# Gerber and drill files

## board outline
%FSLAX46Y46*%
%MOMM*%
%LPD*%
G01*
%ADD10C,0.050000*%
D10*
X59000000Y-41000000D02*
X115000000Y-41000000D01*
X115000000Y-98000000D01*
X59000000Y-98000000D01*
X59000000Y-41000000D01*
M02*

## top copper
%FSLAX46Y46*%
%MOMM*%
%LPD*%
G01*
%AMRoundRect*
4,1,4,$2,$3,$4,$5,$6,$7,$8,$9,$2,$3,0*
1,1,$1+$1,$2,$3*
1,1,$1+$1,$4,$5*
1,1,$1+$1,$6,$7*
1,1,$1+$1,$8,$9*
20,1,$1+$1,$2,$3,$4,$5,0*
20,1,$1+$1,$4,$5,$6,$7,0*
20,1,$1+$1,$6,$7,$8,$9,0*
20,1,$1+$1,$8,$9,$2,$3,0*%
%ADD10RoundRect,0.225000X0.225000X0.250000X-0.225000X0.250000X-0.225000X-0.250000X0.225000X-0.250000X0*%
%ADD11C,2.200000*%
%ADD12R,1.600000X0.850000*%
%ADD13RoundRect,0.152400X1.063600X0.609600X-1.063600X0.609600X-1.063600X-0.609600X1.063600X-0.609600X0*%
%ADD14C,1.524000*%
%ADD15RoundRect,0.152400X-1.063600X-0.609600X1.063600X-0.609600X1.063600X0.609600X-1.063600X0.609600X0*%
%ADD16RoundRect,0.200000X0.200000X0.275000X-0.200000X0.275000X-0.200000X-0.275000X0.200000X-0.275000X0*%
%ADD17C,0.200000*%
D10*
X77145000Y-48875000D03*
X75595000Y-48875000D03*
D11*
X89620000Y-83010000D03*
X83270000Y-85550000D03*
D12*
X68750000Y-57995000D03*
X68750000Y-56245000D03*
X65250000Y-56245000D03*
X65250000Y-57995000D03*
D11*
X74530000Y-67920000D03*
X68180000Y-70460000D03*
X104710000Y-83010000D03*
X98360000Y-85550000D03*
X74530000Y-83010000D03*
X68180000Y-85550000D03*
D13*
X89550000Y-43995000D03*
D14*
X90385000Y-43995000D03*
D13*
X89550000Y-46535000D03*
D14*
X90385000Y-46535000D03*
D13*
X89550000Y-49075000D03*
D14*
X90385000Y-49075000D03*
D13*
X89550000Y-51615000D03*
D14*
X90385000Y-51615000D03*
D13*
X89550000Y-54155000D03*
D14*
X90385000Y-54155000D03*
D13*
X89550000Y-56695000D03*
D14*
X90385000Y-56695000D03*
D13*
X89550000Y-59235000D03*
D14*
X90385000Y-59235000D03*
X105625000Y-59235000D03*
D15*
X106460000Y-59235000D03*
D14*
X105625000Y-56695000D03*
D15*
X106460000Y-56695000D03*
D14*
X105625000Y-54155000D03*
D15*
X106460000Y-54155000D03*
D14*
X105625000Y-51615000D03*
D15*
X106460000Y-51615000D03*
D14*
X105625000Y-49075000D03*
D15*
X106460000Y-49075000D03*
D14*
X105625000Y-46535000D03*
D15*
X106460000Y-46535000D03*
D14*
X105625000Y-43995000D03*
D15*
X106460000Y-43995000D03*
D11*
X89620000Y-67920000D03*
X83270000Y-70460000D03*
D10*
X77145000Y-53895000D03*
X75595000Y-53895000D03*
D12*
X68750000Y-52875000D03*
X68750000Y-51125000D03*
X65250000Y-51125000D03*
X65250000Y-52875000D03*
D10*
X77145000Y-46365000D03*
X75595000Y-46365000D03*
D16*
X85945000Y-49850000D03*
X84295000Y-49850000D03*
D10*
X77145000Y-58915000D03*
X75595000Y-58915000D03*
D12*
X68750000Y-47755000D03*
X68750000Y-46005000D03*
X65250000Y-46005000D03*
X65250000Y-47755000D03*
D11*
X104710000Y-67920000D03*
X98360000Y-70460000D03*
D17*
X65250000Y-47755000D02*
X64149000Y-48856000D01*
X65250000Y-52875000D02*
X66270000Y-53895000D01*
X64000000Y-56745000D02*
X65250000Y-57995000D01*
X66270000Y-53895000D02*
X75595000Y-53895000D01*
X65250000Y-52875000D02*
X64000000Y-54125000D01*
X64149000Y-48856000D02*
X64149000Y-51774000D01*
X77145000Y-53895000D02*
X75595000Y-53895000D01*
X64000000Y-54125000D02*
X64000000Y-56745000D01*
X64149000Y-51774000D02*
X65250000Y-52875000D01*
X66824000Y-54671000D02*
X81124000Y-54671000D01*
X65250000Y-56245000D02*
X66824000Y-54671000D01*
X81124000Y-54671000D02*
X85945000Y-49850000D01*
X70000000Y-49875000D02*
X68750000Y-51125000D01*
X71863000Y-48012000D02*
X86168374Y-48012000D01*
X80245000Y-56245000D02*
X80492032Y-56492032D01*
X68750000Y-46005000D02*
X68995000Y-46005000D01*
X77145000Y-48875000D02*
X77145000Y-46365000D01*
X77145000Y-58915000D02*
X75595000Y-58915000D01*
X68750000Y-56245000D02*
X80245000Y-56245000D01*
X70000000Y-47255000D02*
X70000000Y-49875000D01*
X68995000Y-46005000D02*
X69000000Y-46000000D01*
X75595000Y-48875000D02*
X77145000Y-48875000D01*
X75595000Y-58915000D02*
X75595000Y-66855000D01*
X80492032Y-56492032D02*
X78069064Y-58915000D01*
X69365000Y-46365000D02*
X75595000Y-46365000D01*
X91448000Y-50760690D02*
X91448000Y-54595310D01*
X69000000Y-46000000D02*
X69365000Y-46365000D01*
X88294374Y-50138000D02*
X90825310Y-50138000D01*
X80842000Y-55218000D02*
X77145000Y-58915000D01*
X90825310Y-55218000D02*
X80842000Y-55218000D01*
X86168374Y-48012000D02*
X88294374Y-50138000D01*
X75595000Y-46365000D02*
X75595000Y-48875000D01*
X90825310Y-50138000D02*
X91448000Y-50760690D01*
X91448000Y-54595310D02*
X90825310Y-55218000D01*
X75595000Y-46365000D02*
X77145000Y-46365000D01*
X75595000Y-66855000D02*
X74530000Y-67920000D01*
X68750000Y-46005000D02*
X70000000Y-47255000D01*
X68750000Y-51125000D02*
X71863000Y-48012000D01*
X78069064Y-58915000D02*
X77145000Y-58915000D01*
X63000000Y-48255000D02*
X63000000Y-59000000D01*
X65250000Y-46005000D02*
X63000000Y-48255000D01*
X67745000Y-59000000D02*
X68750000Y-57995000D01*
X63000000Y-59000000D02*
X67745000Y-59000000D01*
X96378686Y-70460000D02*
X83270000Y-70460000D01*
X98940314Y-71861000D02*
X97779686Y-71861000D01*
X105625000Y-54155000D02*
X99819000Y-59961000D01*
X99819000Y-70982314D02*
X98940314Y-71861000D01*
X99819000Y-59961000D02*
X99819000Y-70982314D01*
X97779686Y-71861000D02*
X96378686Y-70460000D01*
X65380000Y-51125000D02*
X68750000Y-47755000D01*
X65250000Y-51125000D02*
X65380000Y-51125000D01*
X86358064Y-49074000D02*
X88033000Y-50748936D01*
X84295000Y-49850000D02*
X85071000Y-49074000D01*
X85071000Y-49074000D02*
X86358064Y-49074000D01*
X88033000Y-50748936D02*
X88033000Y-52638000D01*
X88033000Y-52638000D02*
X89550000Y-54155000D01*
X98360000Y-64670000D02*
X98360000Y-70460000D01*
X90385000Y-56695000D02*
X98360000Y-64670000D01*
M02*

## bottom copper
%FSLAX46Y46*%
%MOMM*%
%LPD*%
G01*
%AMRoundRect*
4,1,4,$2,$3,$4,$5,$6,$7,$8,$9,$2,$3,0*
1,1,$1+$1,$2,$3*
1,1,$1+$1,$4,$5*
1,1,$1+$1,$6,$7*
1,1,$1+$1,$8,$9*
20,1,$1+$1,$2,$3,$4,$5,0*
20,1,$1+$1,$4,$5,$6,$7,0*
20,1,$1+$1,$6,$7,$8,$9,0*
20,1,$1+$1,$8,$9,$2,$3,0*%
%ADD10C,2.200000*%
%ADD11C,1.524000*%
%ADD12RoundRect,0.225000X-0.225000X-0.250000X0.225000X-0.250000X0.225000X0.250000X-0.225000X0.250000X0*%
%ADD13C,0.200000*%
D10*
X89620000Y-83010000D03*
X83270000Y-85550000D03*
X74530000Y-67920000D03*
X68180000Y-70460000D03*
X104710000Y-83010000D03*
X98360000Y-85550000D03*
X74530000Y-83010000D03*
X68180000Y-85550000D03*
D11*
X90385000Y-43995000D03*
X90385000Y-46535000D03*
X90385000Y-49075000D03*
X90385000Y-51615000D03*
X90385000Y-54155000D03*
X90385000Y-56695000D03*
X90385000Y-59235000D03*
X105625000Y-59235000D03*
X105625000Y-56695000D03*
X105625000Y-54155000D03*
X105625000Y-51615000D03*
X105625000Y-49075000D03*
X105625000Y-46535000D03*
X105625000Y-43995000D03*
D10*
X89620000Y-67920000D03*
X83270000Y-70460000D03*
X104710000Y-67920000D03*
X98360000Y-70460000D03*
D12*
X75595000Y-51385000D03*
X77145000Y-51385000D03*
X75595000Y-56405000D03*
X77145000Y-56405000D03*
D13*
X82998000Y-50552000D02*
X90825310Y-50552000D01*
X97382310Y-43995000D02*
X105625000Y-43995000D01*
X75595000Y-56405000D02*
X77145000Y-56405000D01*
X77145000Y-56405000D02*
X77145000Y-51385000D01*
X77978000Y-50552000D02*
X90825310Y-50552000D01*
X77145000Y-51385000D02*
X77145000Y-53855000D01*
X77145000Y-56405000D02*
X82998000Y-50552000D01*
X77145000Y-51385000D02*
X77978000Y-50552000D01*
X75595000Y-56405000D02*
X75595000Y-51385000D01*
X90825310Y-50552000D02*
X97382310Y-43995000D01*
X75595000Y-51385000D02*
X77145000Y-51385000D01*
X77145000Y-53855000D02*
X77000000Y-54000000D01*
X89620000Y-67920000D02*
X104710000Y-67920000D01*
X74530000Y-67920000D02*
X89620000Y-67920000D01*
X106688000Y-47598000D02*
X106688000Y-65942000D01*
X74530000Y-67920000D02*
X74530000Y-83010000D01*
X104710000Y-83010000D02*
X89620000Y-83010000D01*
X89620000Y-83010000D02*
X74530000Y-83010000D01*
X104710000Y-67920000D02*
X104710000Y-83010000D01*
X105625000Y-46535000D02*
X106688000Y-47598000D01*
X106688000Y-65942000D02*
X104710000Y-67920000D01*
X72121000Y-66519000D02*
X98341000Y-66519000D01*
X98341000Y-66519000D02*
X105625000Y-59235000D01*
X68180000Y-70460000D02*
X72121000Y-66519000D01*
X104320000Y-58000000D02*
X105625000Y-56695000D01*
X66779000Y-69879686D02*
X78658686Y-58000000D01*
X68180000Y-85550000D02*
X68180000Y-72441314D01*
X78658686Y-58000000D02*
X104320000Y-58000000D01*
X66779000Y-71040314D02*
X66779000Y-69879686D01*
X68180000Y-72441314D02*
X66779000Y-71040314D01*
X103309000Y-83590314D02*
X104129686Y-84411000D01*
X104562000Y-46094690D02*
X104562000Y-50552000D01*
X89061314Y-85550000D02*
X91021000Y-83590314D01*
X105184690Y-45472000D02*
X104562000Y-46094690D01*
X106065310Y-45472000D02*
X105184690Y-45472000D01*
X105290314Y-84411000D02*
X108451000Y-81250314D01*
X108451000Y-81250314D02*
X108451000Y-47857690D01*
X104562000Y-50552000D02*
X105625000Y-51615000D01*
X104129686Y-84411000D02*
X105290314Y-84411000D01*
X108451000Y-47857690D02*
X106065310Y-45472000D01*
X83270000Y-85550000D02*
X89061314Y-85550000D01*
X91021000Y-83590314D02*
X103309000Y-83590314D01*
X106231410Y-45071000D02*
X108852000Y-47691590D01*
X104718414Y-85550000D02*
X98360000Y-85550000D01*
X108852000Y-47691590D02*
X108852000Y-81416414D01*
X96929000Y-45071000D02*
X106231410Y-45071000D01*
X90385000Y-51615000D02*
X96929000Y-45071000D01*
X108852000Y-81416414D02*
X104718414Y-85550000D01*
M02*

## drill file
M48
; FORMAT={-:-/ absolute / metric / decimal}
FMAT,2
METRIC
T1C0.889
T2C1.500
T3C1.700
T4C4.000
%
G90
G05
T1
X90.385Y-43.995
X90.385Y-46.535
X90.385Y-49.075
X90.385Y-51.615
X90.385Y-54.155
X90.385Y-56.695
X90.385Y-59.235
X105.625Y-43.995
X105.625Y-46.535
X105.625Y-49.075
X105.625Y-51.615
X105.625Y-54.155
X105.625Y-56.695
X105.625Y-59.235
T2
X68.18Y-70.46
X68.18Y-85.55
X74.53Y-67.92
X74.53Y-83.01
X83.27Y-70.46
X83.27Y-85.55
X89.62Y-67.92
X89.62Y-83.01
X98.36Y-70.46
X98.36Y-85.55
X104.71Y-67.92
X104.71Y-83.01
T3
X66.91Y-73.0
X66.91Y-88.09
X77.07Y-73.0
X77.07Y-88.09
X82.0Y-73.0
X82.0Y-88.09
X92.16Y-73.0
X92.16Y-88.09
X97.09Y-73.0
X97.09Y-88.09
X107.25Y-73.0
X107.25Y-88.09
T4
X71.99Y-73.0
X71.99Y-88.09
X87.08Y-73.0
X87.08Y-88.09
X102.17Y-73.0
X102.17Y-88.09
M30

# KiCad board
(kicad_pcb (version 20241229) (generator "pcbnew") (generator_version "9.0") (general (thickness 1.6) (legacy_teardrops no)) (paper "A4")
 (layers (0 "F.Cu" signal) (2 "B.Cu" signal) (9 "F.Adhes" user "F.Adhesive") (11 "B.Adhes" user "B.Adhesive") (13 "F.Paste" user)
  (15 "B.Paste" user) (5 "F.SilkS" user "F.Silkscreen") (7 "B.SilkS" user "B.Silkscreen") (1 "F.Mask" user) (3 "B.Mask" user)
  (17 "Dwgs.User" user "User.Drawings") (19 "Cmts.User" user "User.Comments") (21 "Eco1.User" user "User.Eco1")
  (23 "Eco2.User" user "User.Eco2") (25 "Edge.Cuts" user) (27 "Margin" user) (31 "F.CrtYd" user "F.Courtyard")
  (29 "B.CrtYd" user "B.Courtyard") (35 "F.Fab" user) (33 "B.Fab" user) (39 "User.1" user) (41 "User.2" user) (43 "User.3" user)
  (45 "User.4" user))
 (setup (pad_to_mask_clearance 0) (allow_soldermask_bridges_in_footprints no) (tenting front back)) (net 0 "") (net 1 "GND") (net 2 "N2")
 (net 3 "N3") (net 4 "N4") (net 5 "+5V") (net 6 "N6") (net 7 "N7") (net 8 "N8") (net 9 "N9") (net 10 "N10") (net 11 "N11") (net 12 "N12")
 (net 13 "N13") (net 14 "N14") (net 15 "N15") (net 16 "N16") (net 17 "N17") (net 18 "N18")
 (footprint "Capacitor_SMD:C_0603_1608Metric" (layer "F.Cu") (at 76.37 48.875 180)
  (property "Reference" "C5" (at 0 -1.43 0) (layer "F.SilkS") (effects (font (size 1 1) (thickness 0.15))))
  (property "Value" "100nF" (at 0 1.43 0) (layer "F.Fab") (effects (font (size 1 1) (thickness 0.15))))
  (pad "1" smd roundrect (at -0.775 0 180) (size 0.9 0.95) (layers "F.Cu" "F.Mask" "F.Paste") (roundrect_rratio 0.25) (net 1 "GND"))
  (pad "2" smd roundrect (at 0.775 0 180) (size 0.9 0.95) (layers "F.Cu" "F.Mask" "F.Paste") (roundrect_rratio 0.25) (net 1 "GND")))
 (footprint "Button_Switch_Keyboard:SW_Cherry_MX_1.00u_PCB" (layer "F.Cu") (at 89.62 83.01)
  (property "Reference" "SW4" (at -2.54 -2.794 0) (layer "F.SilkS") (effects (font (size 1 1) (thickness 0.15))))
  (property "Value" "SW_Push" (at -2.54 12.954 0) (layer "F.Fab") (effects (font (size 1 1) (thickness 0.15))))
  (pad "" np_thru_hole circle (at -7.62 5.08) (size 1.7 1.7) (drill 1.7) (layers "*.Cu" "*.Mask"))
  (pad "" np_thru_hole circle (at -2.54 5.08) (size 4 4) (drill 4) (layers "*.Cu" "*.Mask"))
  (pad "" np_thru_hole circle (at 2.54 5.08) (size 1.7 1.7) (drill 1.7) (layers "*.Cu" "*.Mask"))
  (pad "1" thru_hole circle (at 0 0) (size 2.2 2.2) (drill 1.5) (layers "*.Cu" "*.Mask") (remove_unused_layers no) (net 1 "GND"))
  (pad "2" thru_hole circle (at -6.35 2.54) (size 2.2 2.2) (drill 1.5) (layers "*.Cu" "*.Mask") (remove_unused_layers no) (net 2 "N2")))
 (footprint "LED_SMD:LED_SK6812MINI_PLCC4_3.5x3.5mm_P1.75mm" (layer "F.Cu") (at 67 57.12 180)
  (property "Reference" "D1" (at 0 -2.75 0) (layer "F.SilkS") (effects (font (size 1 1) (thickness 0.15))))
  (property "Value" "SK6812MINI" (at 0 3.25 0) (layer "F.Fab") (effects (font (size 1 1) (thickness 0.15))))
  (pad "1" smd rect (at -1.75 -0.875 180) (size 1.6 0.85) (layers "F.Cu" "F.Mask" "F.Paste") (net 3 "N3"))
  (pad "2" smd rect (at -1.75 0.875 180) (size 1.6 0.85) (layers "F.Cu" "F.Mask" "F.Paste") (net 1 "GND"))
  (pad "3" smd rect (at 1.75 0.875 180) (size 1.6 0.85) (layers "F.Cu" "F.Mask" "F.Paste") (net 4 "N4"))
  (pad "4" smd rect (at 1.75 -0.875 180) (size 1.6 0.85) (layers "F.Cu" "F.Mask" "F.Paste") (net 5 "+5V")))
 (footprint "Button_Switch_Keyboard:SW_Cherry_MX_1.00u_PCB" (layer "F.Cu") (at 74.53 67.92)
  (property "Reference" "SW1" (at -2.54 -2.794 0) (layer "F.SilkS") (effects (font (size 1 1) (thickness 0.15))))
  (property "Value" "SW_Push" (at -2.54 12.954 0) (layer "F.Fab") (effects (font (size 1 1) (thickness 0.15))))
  (pad "" np_thru_hole circle (at -7.62 5.08) (size 1.7 1.7) (drill 1.7) (layers "*.Cu" "*.Mask"))
  (pad "" np_thru_hole circle (at -2.54 5.08) (size 4 4) (drill 4) (layers "*.Cu" "*.Mask"))
  (pad "" np_thru_hole circle (at 2.54 5.08) (size 1.7 1.7) (drill 1.7) (layers "*.Cu" "*.Mask"))
  (pad "1" thru_hole circle (at 0 0) (size 2.2 2.2) (drill 1.5) (layers "*.Cu" "*.Mask") (remove_unused_layers no) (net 1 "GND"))
  (pad "2" thru_hole circle (at -6.35 2.54) (size 2.2 2.2) (drill 1.5) (layers "*.Cu" "*.Mask") (remove_unused_layers no) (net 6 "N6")))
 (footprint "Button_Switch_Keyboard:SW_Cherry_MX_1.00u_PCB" (layer "F.Cu") (at 104.71 83.01)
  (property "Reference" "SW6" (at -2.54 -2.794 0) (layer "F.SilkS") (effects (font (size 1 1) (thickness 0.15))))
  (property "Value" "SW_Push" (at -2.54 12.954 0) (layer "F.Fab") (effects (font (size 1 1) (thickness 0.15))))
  (pad "" np_thru_hole circle (at -7.62 5.08) (size 1.7 1.7) (drill 1.7) (layers "*.Cu" "*.Mask"))
  (pad "" np_thru_hole circle (at -2.54 5.08) (size 4 4) (drill 4) (layers "*.Cu" "*.Mask"))
  (pad "" np_thru_hole circle (at 2.54 5.08) (size 1.7 1.7) (drill 1.7) (layers "*.Cu" "*.Mask"))
  (pad "1" thru_hole circle (at 0 0) (size 2.2 2.2) (drill 1.5) (layers "*.Cu" "*.Mask") (remove_unused_layers no) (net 1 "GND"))
  (pad "2" thru_hole circle (at -6.35 2.54) (size 2.2 2.2) (drill 1.5) (layers "*.Cu" "*.Mask") (remove_unused_layers no) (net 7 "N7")))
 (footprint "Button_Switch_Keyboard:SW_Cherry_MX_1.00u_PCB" (layer "F.Cu") (at 74.53 83.01)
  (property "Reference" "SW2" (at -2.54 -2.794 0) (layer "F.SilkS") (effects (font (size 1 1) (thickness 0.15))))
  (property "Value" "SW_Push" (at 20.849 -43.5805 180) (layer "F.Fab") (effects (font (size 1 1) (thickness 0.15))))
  (pad "" np_thru_hole circle (at -7.62 5.08) (size 1.7 1.7) (drill 1.7) (layers "*.Cu" "*.Mask"))
  (pad "" np_thru_hole circle (at -2.54 5.08) (size 4 4) (drill 4) (layers "*.Cu" "*.Mask"))
  (pad "" np_thru_hole circle (at 2.54 5.08) (size 1.7 1.7) (drill 1.7) (layers "*.Cu" "*.Mask"))
  (pad "1" thru_hole circle (at 0 0) (size 2.2 2.2) (drill 1.5) (layers "*.Cu" "*.Mask") (remove_unused_layers no) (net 1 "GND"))
  (pad "2" thru_hole circle (at -6.35 2.54) (size 2.2 2.2) (drill 1.5) (layers "*.Cu" "*.Mask") (remove_unused_layers no) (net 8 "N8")))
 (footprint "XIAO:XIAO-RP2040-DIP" (layer "F.Cu") (at 98.005 51.615)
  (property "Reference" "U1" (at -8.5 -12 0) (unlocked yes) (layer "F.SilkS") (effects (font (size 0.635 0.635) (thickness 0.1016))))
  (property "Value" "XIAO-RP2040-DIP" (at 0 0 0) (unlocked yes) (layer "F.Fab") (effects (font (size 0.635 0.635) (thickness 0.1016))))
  (pad "1" smd roundrect (at -8.455 -7.62 180) (size 2.432 1.524) (layers "F.Cu" "F.Mask") (roundrect_rratio 0.1) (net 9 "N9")
   (thermal_bridge_angle 45))
  (pad "1" thru_hole circle (at -7.62 -7.62 180) (size 1.524 1.524) (drill 0.889) (layers "*.Cu" "*.Mask") (remove_unused_layers no)
   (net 9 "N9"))
  (pad "2" smd roundrect (at -8.455 -5.08 180) (size 2.432 1.524) (layers "F.Cu" "F.Mask") (roundrect_rratio 0.1) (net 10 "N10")
   (thermal_bridge_angle 45))
  (pad "2" thru_hole circle (at -7.62 -5.08 180) (size 1.524 1.524) (drill 0.889) (layers "*.Cu" "*.Mask") (remove_unused_layers no)
   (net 10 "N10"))
  (pad "3" smd roundrect (at -8.455 -2.54 180) (size 2.432 1.524) (layers "F.Cu" "F.Mask") (roundrect_rratio 0.1) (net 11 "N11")
   (thermal_bridge_angle 45))
  (pad "3" thru_hole circle (at -7.62 -2.54 180) (size 1.524 1.524) (drill 0.889) (layers "*.Cu" "*.Mask") (remove_unused_layers no)
   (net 11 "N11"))
  (pad "4" smd roundrect (at -8.455 0 180) (size 2.432 1.524) (layers "F.Cu" "F.Mask") (roundrect_rratio 0.1) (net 7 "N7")
   (thermal_bridge_angle 45))
  (pad "4" thru_hole circle (at -7.62 0 180) (size 1.524 1.524) (drill 0.889) (layers "*.Cu" "*.Mask") (remove_unused_layers no)
   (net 7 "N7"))
  (pad "5" smd roundrect (at -8.455 2.54 180) (size 2.432 1.524) (layers "F.Cu" "F.Mask") (roundrect_rratio 0.1) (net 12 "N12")
   (thermal_bridge_angle 45))
  (pad "5" thru_hole circle (at -7.62 2.54 180) (size 1.524 1.524) (drill 0.889) (layers "*.Cu" "*.Mask") (remove_unused_layers no)
   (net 12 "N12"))
  (pad "6" smd roundrect (at -8.455 5.08 180) (size 2.432 1.524) (layers "F.Cu" "F.Mask") (roundrect_rratio 0.1) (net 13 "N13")
   (thermal_bridge_angle 45))
  (pad "6" thru_hole circle (at -7.62 5.08 180) (size 1.524 1.524) (drill 0.889) (layers "*.Cu" "*.Mask") (remove_unused_layers no)
   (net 13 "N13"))
  (pad "7" smd roundrect (at -8.455 7.62 180) (size 2.432 1.524) (layers "F.Cu" "F.Mask") (roundrect_rratio 0.1) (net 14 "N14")
   (thermal_bridge_angle 45))
  (pad "7" thru_hole circle (at -7.62 7.62 180) (size 1.524 1.524) (drill 0.889) (layers "*.Cu" "*.Mask") (remove_unused_layers no)
   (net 14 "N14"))
  (pad "8" thru_hole circle (at 7.62 7.62) (size 1.524 1.524) (drill 0.889) (layers "*.Cu" "*.Mask") (remove_unused_layers no) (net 6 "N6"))
  (pad "8" smd roundrect (at 8.455 7.62) (size 2.432 1.524) (layers "F.Cu" "F.Mask") (roundrect_rratio 0.1) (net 6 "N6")
   (thermal_bridge_angle 45))
  (pad "9" thru_hole circle (at 7.62 5.08) (size 1.524 1.524) (drill 0.889) (layers "*.Cu" "*.Mask") (remove_unused_layers no) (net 8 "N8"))
  (pad "9" smd roundrect (at 8.455 5.08) (size 2.432 1.524) (layers "F.Cu" "F.Mask") (roundrect_rratio 0.1) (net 8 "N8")
   (thermal_bridge_angle 45))
  (pad "10" thru_hole circle (at 7.62 2.54) (size 1.524 1.524) (drill 0.889) (layers "*.Cu" "*.Mask") (remove_unused_layers no)
   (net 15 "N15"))
  (pad "10" smd roundrect (at 8.455 2.54) (size 2.432 1.524) (layers "F.Cu" "F.Mask") (roundrect_rratio 0.1) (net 15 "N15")
   (thermal_bridge_angle 45))
  (pad "11" thru_hole circle (at 7.62 0) (size 1.524 1.524) (drill 0.889) (layers "*.Cu" "*.Mask") (remove_unused_layers no) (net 2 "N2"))
  (pad "11" smd roundrect (at 8.455 0) (size 2.432 1.524) (layers "F.Cu" "F.Mask") (roundrect_rratio 0.1) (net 2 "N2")
   (thermal_bridge_angle 45))
  (pad "12" thru_hole circle (at 7.62 -2.54) (size 1.524 1.524) (drill 0.889) (layers "*.Cu" "*.Mask") (remove_unused_layers no)
   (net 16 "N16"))
  (pad "12" smd roundrect (at 8.455 -2.54) (size 2.432 1.524) (layers "F.Cu" "F.Mask") (roundrect_rratio 0.1) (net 16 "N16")
   (thermal_bridge_angle 45))
  (pad "13" thru_hole circle (at 7.62 -5.08) (size 1.524 1.524) (drill 0.889) (layers "*.Cu" "*.Mask") (remove_unused_layers no)
   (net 1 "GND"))
  (pad "13" smd roundrect (at 8.455 -5.08) (size 2.432 1.524) (layers "F.Cu" "F.Mask") (roundrect_rratio 0.1) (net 1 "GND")
   (thermal_bridge_angle 45))
  (pad "14" thru_hole circle (at 7.62 -7.62) (size 1.524 1.524) (drill 0.889) (layers "*.Cu" "*.Mask") (remove_unused_layers no)
   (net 5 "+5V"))
  (pad "14" smd roundrect (at 8.455 -7.62) (size 2.432 1.524) (layers "F.Cu" "F.Mask") (roundrect_rratio 0.1) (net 5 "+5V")
   (thermal_bridge_angle 45)))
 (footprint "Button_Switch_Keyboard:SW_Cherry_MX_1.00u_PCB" (layer "F.Cu") (at 89.62 67.92)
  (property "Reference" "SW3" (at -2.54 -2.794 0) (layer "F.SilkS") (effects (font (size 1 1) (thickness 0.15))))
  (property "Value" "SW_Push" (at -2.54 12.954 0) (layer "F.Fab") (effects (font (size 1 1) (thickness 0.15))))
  (pad "" np_thru_hole circle (at -7.62 5.08) (size 1.7 1.7) (drill 1.7) (layers "*.Cu" "*.Mask"))
  (pad "" np_thru_hole circle (at -2.54 5.08) (size 4 4) (drill 4) (layers "*.Cu" "*.Mask"))
  (pad "" np_thru_hole circle (at 2.54 5.08) (size 1.7 1.7) (drill 1.7) (layers "*.Cu" "*.Mask"))
  (pad "1" thru_hole circle (at 0 0) (size 2.2 2.2) (drill 1.5) (layers "*.Cu" "*.Mask") (remove_unused_layers no) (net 1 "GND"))
  (pad "2" thru_hole circle (at -6.35 2.54) (size 2.2 2.2) (drill 1.5) (layers "*.Cu" "*.Mask") (remove_unused_layers no) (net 15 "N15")))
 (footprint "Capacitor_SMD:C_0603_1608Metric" (layer "F.Cu") (at 76.37 53.895 180)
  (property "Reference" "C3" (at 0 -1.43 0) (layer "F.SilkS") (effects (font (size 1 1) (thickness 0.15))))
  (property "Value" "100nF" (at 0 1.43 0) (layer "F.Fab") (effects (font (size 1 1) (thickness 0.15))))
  (pad "1" smd roundrect (at -0.775 0 180) (size 0.9 0.95) (layers "F.Cu" "F.Mask" "F.Paste") (roundrect_rratio 0.25) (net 5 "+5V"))
  (pad "2" smd roundrect (at 0.775 0 180) (size 0.9 0.95) (layers "F.Cu" "F.Mask" "F.Paste") (roundrect_rratio 0.25) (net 5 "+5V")))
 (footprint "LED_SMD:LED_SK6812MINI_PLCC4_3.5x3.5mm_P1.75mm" (layer "F.Cu") (at 67 52 180)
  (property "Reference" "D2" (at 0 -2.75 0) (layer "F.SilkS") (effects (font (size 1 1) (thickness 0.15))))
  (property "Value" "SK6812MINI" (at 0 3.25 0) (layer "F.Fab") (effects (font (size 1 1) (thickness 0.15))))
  (pad "1" smd rect (at -1.75 -0.875 180) (size 1.6 0.85) (layers "F.Cu" "F.Mask" "F.Paste") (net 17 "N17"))
  (pad "2" smd rect (at -1.75 0.875 180) (size 1.6 0.85) (layers "F.Cu" "F.Mask" "F.Paste") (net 1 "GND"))
  (pad "3" smd rect (at 1.75 0.875 180) (size 1.6 0.85) (layers "F.Cu" "F.Mask" "F.Paste") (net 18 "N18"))
  (pad "4" smd rect (at 1.75 -0.875 180) (size 1.6 0.85) (layers "F.Cu" "F.Mask" "F.Paste") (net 5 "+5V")))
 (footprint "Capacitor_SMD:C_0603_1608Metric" (layer "F.Cu") (at 76.37 46.365 180)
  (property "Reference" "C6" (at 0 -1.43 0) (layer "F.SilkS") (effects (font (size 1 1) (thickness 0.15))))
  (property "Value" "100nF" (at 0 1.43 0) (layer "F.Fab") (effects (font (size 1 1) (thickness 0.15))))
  (pad "1" smd roundrect (at -0.775 0 180) (size 0.9 0.95) (layers "F.Cu" "F.Mask" "F.Paste") (roundrect_rratio 0.25) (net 1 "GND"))
  (pad "2" smd roundrect (at 0.775 0 180) (size 0.9 0.95) (layers "F.Cu" "F.Mask" "F.Paste") (roundrect_rratio 0.25) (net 1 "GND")))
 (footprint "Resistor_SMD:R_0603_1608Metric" (layer "F.Cu") (at 85.12 49.85 180)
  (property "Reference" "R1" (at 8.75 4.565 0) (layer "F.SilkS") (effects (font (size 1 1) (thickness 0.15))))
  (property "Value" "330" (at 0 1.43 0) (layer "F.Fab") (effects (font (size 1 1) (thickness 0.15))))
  (pad "1" smd roundrect (at -0.825 0 180) (size 0.8 0.95) (layers "F.Cu" "F.Mask" "F.Paste") (roundrect_rratio 0.25) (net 4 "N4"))
  (pad "2" smd roundrect (at 0.825 0 180) (size 0.8 0.95) (layers "F.Cu" "F.Mask" "F.Paste") (roundrect_rratio 0.25) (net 12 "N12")))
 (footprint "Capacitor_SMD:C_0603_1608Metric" (layer "F.Cu") (at 76.37 58.915 180)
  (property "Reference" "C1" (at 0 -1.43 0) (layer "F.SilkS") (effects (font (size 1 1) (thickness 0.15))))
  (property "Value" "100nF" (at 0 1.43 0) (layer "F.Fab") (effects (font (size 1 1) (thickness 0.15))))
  (pad "1" smd roundrect (at -0.775 0 180) (size 0.9 0.95) (layers "F.Cu" "F.Mask" "F.Paste") (roundrect_rratio 0.25) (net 1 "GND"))
  (pad "2" smd roundrect (at 0.775 0 180) (size 0.9 0.95) (layers "F.Cu" "F.Mask" "F.Paste") (roundrect_rratio 0.25) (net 1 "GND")))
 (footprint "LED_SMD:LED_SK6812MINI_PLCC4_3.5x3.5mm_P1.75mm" (layer "F.Cu") (at 67 46.88 180)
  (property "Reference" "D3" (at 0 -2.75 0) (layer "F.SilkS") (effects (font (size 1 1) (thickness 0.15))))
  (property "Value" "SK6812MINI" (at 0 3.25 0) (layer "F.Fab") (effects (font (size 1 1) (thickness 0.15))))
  (pad "1" smd rect (at -1.75 -0.875 180) (size 1.6 0.85) (layers "F.Cu" "F.Mask" "F.Paste") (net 18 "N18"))
  (pad "2" smd rect (at -1.75 0.875 180) (size 1.6 0.85) (layers "F.Cu" "F.Mask" "F.Paste") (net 1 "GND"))
  (pad "3" smd rect (at 1.75 0.875 180) (size 1.6 0.85) (layers "F.Cu" "F.Mask" "F.Paste") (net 3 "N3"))
  (pad "4" smd rect (at 1.75 -0.875 180) (size 1.6 0.85) (layers "F.Cu" "F.Mask" "F.Paste") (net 5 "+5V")))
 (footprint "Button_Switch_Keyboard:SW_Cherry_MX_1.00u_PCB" (layer "F.Cu") (at 104.71 67.92)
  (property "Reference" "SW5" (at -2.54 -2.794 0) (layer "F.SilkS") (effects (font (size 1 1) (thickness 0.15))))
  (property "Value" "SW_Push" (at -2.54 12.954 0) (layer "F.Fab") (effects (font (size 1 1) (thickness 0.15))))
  (pad "" np_thru_hole circle (at -7.62 5.08) (size 1.7 1.7) (drill 1.7) (layers "*.Cu" "*.Mask"))
  (pad "" np_thru_hole circle (at -2.54 5.08) (size 4 4) (drill 4) (layers "*.Cu" "*.Mask"))
  (pad "" np_thru_hole circle (at 2.54 5.08) (size 1.7 1.7) (drill 1.7) (layers "*.Cu" "*.Mask"))
  (pad "1" thru_hole circle (at 0 0) (size 2.2 2.2) (drill 1.5) (layers "*.Cu" "*.Mask") (remove_unused_layers no) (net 1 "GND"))
  (pad "2" thru_hole circle (at -6.35 2.54) (size 2.2 2.2) (drill 1.5) (layers "*.Cu" "*.Mask") (remove_unused_layers no) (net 13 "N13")))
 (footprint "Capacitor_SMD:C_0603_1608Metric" (layer "B.Cu") (at 76.37 51.385)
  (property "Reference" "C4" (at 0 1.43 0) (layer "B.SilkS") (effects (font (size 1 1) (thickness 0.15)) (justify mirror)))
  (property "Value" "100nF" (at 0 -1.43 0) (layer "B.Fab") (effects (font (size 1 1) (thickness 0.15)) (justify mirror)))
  (pad "1" smd roundrect (at -0.775 0) (size 0.9 0.95) (layers "B.Cu" "B.Mask" "B.Paste") (roundrect_rratio 0.25) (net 5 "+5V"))
  (pad "2" smd roundrect (at 0.775 0) (size 0.9 0.95) (layers "B.Cu" "B.Mask" "B.Paste") (roundrect_rratio 0.25) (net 5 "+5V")))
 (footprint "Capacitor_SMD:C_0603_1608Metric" (layer "B.Cu") (at 76.37 56.405)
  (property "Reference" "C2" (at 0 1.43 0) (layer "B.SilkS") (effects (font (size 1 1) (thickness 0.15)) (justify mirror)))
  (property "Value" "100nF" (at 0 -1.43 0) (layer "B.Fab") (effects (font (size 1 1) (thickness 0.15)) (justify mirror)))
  (pad "1" smd roundrect (at -0.775 0) (size 0.9 0.95) (layers "B.Cu" "B.Mask" "B.Paste") (roundrect_rratio 0.25) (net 5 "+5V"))
  (pad "2" smd roundrect (at 0.775 0) (size 0.9 0.95) (layers "B.Cu" "B.Mask" "B.Paste") (roundrect_rratio 0.25) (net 5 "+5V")))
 (gr_rect (start 59 41) (end 115 98) (stroke (width 0.05) (type default)) (fill no) (layer "Edge.Cuts"))
 (segment (start 65.25 47.755) (end 64.149 48.856) (width 0.2) (layer "F.Cu") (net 5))
 (segment (start 65.25 52.875) (end 66.27 53.895) (width 0.2) (layer "F.Cu") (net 5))
 (segment (start 64 56.745) (end 65.25 57.995) (width 0.2) (layer "F.Cu") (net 5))
 (segment (start 66.27 53.895) (end 75.595 53.895) (width 0.2) (layer "F.Cu") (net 5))
 (segment (start 65.25 52.875) (end 64 54.125) (width 0.2) (layer "F.Cu") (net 5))
 (segment (start 64.149 48.856) (end 64.149 51.774) (width 0.2) (layer "F.Cu") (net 5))
 (segment (start 77.145 53.895) (end 75.595 53.895) (width 0.2) (layer "F.Cu") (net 5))
 (segment (start 64 54.125) (end 64 56.745) (width 0.2) (layer "F.Cu") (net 5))
 (segment (start 64.149 51.774) (end 65.25 52.875) (width 0.2) (layer "F.Cu") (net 5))
 (segment (start 82.998 50.552) (end 90.82531 50.552) (width 0.2) (layer "B.Cu") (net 5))
 (segment (start 97.38231 43.995) (end 105.625 43.995) (width 0.2) (layer "B.Cu") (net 5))
 (segment (start 75.595 56.405) (end 77.145 56.405) (width 0.2) (layer "B.Cu") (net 5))
 (segment (start 77.145 56.405) (end 77.145 51.385) (width 0.2) (layer "B.Cu") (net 5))
 (segment (start 77.978 50.552) (end 90.82531 50.552) (width 0.2) (layer "B.Cu") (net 5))
 (segment (start 77.145 51.385) (end 77.145 53.855) (width 0.2) (layer "B.Cu") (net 5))
 (segment (start 77.145 56.405) (end 82.998 50.552) (width 0.2) (layer "B.Cu") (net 5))
 (segment (start 77.145 51.385) (end 77.978 50.552) (width 0.2) (layer "B.Cu") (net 5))
 (segment (start 75.595 56.405) (end 75.595 51.385) (width 0.2) (layer "B.Cu") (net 5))
 (segment (start 90.82531 50.552) (end 97.38231 43.995) (width 0.2) (layer "B.Cu") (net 5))
 (segment (start 75.595 51.385) (end 77.145 51.385) (width 0.2) (layer "B.Cu") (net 5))
 (segment (start 77.145 53.855) (end 77 54) (width 0.2) (layer "B.Cu") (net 5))
 (segment (start 66.824 54.671) (end 81.124 54.671) (width 0.2) (layer "F.Cu") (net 4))
 (segment (start 65.25 56.245) (end 66.824 54.671) (width 0.2) (layer "F.Cu") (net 4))
 (segment (start 81.124 54.671) (end 85.945 49.85) (width 0.2) (layer "F.Cu") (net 4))
 (segment (start 70 49.875) (end 68.75 51.125) (width 0.2) (layer "F.Cu") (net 1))
 (segment (start 71.863 48.012) (end 86.168374 48.012) (width 0.2) (layer "F.Cu") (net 1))
 (segment (start 80.245 56.245) (end 80.492032 56.492032) (width 0.2) (layer "F.Cu") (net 1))
 (segment (start 68.75 46.005) (end 68.995 46.005) (width 0.2) (layer "F.Cu") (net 1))
 (segment (start 77.145 48.875) (end 77.145 46.365) (width 0.2) (layer "F.Cu") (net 1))
 (segment (start 77.145 58.915) (end 75.595 58.915) (width 0.2) (layer "F.Cu") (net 1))
 (segment (start 68.75 56.245) (end 80.245 56.245) (width 0.2) (layer "F.Cu") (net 1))
 (segment (start 70 47.255) (end 70 49.875) (width 0.2) (layer "F.Cu") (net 1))
 (segment (start 68.995 46.005) (end 69 46) (width 0.2) (layer "F.Cu") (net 1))
 (segment (start 75.595 48.875) (end 77.145 48.875) (width 0.2) (layer "F.Cu") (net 1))
 (segment (start 75.595 58.915) (end 75.595 66.855) (width 0.2) (layer "F.Cu") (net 1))
 (segment (start 80.492032 56.492032) (end 78.069064 58.915) (width 0.2) (layer "F.Cu") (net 1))
 (segment (start 69.365 46.365) (end 75.595 46.365) (width 0.2) (layer "F.Cu") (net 1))
 (segment (start 91.448 50.76069) (end 91.448 54.59531) (width 0.2) (layer "F.Cu") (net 1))
 (segment (start 69 46) (end 69.365 46.365) (width 0.2) (layer "F.Cu") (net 1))
 (segment (start 88.294374 50.138) (end 90.82531 50.138) (width 0.2) (layer "F.Cu") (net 1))
 (segment (start 80.842 55.218) (end 77.145 58.915) (width 0.2) (layer "F.Cu") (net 1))
 (segment (start 90.82531 55.218) (end 80.842 55.218) (width 0.2) (layer "F.Cu") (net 1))
 (segment (start 86.168374 48.012) (end 88.294374 50.138) (width 0.2) (layer "F.Cu") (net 1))
 (segment (start 75.595 46.365) (end 75.595 48.875) (width 0.2) (layer "F.Cu") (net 1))
 (segment (start 90.82531 50.138) (end 91.448 50.76069) (width 0.2) (layer "F.Cu") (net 1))
 (segment (start 91.448 54.59531) (end 90.82531 55.218) (width 0.2) (layer "F.Cu") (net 1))
 (segment (start 75.595 46.365) (end 77.145 46.365) (width 0.2) (layer "F.Cu") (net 1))
 (segment (start 75.595 66.855) (end 74.53 67.92) (width 0.2) (layer "F.Cu") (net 1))
 (segment (start 68.75 46.005) (end 70 47.255) (width 0.2) (layer "F.Cu") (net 1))
 (segment (start 68.75 51.125) (end 71.863 48.012) (width 0.2) (layer "F.Cu") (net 1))
 (segment (start 78.069064 58.915) (end 77.145 58.915) (width 0.2) (layer "F.Cu") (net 1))
 (segment (start 89.62 67.92) (end 104.71 67.92) (width 0.2) (layer "B.Cu") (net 1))
 (segment (start 74.53 67.92) (end 89.62 67.92) (width 0.2) (layer "B.Cu") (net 1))
 (segment (start 106.688 47.598) (end 106.688 65.942) (width 0.2) (layer "B.Cu") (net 1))
 (segment (start 74.53 67.92) (end 74.53 83.01) (width 0.2) (layer "B.Cu") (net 1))
 (segment (start 104.71 83.01) (end 89.62 83.01) (width 0.2) (layer "B.Cu") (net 1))
 (segment (start 89.62 83.01) (end 74.53 83.01) (width 0.2) (layer "B.Cu") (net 1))
 (segment (start 104.71 67.92) (end 104.71 83.01) (width 0.2) (layer "B.Cu") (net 1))
 (segment (start 105.625 46.535) (end 106.688 47.598) (width 0.2) (layer "B.Cu") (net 1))
 (segment (start 106.688 65.942) (end 104.71 67.92) (width 0.2) (layer "B.Cu") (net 1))
 (segment (start 63 48.255) (end 63 59) (width 0.2) (layer "F.Cu") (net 3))
 (segment (start 65.25 46.005) (end 63 48.255) (width 0.2) (layer "F.Cu") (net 3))
 (segment (start 67.745 59) (end 68.75 57.995) (width 0.2) (layer "F.Cu") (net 3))
 (segment (start 63 59) (end 67.745 59) (width 0.2) (layer "F.Cu") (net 3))
 (segment (start 72.121 66.519) (end 98.341 66.519) (width 0.2) (layer "B.Cu") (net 6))
 (segment (start 98.341 66.519) (end 105.625 59.235) (width 0.2) (layer "B.Cu") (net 6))
 (segment (start 68.18 70.46) (end 72.121 66.519) (width 0.2) (layer "B.Cu") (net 6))
 (segment (start 104.32 58) (end 105.625 56.695) (width 0.2) (layer "B.Cu") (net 8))
 (segment (start 66.779 69.879686) (end 78.658686 58) (width 0.2) (layer "B.Cu") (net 8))
 (segment (start 68.18 85.55) (end 68.18 72.441314) (width 0.2) (layer "B.Cu") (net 8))
 (segment (start 78.658686 58) (end 104.32 58) (width 0.2) (layer "B.Cu") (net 8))
 (segment (start 66.779 71.040314) (end 66.779 69.879686) (width 0.2) (layer "B.Cu") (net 8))
 (segment (start 68.18 72.441314) (end 66.779 71.040314) (width 0.2) (layer "B.Cu") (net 8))
 (segment (start 96.378686 70.46) (end 83.27 70.46) (width 0.2) (layer "F.Cu") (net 15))
 (segment (start 98.940314 71.861) (end 97.779686 71.861) (width 0.2) (layer "F.Cu") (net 15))
 (segment (start 105.625 54.155) (end 99.819 59.961) (width 0.2) (layer "F.Cu") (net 15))
 (segment (start 99.819 70.982314) (end 98.940314 71.861) (width 0.2) (layer "F.Cu") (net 15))
 (segment (start 99.819 59.961) (end 99.819 70.982314) (width 0.2) (layer "F.Cu") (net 15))
 (segment (start 97.779686 71.861) (end 96.378686 70.46) (width 0.2) (layer "F.Cu") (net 15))
 (segment (start 103.309 83.590314) (end 104.129686 84.411) (width 0.2) (layer "B.Cu") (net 2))
 (segment (start 104.562 46.09469) (end 104.562 50.552) (width 0.2) (layer "B.Cu") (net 2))
 (segment (start 89.061314 85.55) (end 91.021 83.590314) (width 0.2) (layer "B.Cu") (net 2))
 (segment (start 105.18469 45.472) (end 104.562 46.09469) (width 0.2) (layer "B.Cu") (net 2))
 (segment (start 106.06531 45.472) (end 105.18469 45.472) (width 0.2) (layer "B.Cu") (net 2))
 (segment (start 105.290314 84.411) (end 108.451 81.250314) (width 0.2) (layer "B.Cu") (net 2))
 (segment (start 108.451 81.250314) (end 108.451 47.85769) (width 0.2) (layer "B.Cu") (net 2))
 (segment (start 104.562 50.552) (end 105.625 51.615) (width 0.2) (layer "B.Cu") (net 2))
 (segment (start 104.129686 84.411) (end 105.290314 84.411) (width 0.2) (layer "B.Cu") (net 2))
 (segment (start 108.451 47.85769) (end 106.06531 45.472) (width 0.2) (layer "B.Cu") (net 2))
 (segment (start 83.27 85.55) (end 89.061314 85.55) (width 0.2) (layer "B.Cu") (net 2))
 (segment (start 91.021 83.590314) (end 103.309 83.590314) (width 0.2) (layer "B.Cu") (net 2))
 (segment (start 65.38 51.125) (end 68.75 47.755) (width 0.2) (layer "F.Cu") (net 18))
 (segment (start 65.25 51.125) (end 65.38 51.125) (width 0.2) (layer "F.Cu") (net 18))
 (segment (start 86.358064 49.074) (end 88.033 50.748936) (width 0.2) (layer "F.Cu") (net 12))
 (segment (start 84.295 49.85) (end 85.071 49.074) (width 0.2) (layer "F.Cu") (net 12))
 (segment (start 85.071 49.074) (end 86.358064 49.074) (width 0.2) (layer "F.Cu") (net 12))
 (segment (start 88.033 50.748936) (end 88.033 52.638) (width 0.2) (layer "F.Cu") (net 12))
 (segment (start 88.033 52.638) (end 89.55 54.155) (width 0.2) (layer "F.Cu") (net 12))
 (segment (start 98.36 64.67) (end 98.36 70.46) (width 0.2) (layer "F.Cu") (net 13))
 (segment (start 90.385 56.695) (end 98.36 64.67) (width 0.2) (layer "F.Cu") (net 13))
 (segment (start 106.23141 45.071) (end 108.852 47.69159) (width 0.2) (layer "B.Cu") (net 7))
 (segment (start 104.718414 85.55) (end 98.36 85.55) (width 0.2) (layer "B.Cu") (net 7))
 (segment (start 108.852 47.69159) (end 108.852 81.416414) (width 0.2) (layer "B.Cu") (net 7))
 (segment (start 96.929 45.071) (end 106.23141 45.071) (width 0.2) (layer "B.Cu") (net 7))
 (segment (start 90.385 51.615) (end 96.929 45.071) (width 0.2) (layer "B.Cu") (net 7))
 (segment (start 108.852 81.416414) (end 104.718414 85.55) (width 0.2) (layer "B.Cu") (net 7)))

